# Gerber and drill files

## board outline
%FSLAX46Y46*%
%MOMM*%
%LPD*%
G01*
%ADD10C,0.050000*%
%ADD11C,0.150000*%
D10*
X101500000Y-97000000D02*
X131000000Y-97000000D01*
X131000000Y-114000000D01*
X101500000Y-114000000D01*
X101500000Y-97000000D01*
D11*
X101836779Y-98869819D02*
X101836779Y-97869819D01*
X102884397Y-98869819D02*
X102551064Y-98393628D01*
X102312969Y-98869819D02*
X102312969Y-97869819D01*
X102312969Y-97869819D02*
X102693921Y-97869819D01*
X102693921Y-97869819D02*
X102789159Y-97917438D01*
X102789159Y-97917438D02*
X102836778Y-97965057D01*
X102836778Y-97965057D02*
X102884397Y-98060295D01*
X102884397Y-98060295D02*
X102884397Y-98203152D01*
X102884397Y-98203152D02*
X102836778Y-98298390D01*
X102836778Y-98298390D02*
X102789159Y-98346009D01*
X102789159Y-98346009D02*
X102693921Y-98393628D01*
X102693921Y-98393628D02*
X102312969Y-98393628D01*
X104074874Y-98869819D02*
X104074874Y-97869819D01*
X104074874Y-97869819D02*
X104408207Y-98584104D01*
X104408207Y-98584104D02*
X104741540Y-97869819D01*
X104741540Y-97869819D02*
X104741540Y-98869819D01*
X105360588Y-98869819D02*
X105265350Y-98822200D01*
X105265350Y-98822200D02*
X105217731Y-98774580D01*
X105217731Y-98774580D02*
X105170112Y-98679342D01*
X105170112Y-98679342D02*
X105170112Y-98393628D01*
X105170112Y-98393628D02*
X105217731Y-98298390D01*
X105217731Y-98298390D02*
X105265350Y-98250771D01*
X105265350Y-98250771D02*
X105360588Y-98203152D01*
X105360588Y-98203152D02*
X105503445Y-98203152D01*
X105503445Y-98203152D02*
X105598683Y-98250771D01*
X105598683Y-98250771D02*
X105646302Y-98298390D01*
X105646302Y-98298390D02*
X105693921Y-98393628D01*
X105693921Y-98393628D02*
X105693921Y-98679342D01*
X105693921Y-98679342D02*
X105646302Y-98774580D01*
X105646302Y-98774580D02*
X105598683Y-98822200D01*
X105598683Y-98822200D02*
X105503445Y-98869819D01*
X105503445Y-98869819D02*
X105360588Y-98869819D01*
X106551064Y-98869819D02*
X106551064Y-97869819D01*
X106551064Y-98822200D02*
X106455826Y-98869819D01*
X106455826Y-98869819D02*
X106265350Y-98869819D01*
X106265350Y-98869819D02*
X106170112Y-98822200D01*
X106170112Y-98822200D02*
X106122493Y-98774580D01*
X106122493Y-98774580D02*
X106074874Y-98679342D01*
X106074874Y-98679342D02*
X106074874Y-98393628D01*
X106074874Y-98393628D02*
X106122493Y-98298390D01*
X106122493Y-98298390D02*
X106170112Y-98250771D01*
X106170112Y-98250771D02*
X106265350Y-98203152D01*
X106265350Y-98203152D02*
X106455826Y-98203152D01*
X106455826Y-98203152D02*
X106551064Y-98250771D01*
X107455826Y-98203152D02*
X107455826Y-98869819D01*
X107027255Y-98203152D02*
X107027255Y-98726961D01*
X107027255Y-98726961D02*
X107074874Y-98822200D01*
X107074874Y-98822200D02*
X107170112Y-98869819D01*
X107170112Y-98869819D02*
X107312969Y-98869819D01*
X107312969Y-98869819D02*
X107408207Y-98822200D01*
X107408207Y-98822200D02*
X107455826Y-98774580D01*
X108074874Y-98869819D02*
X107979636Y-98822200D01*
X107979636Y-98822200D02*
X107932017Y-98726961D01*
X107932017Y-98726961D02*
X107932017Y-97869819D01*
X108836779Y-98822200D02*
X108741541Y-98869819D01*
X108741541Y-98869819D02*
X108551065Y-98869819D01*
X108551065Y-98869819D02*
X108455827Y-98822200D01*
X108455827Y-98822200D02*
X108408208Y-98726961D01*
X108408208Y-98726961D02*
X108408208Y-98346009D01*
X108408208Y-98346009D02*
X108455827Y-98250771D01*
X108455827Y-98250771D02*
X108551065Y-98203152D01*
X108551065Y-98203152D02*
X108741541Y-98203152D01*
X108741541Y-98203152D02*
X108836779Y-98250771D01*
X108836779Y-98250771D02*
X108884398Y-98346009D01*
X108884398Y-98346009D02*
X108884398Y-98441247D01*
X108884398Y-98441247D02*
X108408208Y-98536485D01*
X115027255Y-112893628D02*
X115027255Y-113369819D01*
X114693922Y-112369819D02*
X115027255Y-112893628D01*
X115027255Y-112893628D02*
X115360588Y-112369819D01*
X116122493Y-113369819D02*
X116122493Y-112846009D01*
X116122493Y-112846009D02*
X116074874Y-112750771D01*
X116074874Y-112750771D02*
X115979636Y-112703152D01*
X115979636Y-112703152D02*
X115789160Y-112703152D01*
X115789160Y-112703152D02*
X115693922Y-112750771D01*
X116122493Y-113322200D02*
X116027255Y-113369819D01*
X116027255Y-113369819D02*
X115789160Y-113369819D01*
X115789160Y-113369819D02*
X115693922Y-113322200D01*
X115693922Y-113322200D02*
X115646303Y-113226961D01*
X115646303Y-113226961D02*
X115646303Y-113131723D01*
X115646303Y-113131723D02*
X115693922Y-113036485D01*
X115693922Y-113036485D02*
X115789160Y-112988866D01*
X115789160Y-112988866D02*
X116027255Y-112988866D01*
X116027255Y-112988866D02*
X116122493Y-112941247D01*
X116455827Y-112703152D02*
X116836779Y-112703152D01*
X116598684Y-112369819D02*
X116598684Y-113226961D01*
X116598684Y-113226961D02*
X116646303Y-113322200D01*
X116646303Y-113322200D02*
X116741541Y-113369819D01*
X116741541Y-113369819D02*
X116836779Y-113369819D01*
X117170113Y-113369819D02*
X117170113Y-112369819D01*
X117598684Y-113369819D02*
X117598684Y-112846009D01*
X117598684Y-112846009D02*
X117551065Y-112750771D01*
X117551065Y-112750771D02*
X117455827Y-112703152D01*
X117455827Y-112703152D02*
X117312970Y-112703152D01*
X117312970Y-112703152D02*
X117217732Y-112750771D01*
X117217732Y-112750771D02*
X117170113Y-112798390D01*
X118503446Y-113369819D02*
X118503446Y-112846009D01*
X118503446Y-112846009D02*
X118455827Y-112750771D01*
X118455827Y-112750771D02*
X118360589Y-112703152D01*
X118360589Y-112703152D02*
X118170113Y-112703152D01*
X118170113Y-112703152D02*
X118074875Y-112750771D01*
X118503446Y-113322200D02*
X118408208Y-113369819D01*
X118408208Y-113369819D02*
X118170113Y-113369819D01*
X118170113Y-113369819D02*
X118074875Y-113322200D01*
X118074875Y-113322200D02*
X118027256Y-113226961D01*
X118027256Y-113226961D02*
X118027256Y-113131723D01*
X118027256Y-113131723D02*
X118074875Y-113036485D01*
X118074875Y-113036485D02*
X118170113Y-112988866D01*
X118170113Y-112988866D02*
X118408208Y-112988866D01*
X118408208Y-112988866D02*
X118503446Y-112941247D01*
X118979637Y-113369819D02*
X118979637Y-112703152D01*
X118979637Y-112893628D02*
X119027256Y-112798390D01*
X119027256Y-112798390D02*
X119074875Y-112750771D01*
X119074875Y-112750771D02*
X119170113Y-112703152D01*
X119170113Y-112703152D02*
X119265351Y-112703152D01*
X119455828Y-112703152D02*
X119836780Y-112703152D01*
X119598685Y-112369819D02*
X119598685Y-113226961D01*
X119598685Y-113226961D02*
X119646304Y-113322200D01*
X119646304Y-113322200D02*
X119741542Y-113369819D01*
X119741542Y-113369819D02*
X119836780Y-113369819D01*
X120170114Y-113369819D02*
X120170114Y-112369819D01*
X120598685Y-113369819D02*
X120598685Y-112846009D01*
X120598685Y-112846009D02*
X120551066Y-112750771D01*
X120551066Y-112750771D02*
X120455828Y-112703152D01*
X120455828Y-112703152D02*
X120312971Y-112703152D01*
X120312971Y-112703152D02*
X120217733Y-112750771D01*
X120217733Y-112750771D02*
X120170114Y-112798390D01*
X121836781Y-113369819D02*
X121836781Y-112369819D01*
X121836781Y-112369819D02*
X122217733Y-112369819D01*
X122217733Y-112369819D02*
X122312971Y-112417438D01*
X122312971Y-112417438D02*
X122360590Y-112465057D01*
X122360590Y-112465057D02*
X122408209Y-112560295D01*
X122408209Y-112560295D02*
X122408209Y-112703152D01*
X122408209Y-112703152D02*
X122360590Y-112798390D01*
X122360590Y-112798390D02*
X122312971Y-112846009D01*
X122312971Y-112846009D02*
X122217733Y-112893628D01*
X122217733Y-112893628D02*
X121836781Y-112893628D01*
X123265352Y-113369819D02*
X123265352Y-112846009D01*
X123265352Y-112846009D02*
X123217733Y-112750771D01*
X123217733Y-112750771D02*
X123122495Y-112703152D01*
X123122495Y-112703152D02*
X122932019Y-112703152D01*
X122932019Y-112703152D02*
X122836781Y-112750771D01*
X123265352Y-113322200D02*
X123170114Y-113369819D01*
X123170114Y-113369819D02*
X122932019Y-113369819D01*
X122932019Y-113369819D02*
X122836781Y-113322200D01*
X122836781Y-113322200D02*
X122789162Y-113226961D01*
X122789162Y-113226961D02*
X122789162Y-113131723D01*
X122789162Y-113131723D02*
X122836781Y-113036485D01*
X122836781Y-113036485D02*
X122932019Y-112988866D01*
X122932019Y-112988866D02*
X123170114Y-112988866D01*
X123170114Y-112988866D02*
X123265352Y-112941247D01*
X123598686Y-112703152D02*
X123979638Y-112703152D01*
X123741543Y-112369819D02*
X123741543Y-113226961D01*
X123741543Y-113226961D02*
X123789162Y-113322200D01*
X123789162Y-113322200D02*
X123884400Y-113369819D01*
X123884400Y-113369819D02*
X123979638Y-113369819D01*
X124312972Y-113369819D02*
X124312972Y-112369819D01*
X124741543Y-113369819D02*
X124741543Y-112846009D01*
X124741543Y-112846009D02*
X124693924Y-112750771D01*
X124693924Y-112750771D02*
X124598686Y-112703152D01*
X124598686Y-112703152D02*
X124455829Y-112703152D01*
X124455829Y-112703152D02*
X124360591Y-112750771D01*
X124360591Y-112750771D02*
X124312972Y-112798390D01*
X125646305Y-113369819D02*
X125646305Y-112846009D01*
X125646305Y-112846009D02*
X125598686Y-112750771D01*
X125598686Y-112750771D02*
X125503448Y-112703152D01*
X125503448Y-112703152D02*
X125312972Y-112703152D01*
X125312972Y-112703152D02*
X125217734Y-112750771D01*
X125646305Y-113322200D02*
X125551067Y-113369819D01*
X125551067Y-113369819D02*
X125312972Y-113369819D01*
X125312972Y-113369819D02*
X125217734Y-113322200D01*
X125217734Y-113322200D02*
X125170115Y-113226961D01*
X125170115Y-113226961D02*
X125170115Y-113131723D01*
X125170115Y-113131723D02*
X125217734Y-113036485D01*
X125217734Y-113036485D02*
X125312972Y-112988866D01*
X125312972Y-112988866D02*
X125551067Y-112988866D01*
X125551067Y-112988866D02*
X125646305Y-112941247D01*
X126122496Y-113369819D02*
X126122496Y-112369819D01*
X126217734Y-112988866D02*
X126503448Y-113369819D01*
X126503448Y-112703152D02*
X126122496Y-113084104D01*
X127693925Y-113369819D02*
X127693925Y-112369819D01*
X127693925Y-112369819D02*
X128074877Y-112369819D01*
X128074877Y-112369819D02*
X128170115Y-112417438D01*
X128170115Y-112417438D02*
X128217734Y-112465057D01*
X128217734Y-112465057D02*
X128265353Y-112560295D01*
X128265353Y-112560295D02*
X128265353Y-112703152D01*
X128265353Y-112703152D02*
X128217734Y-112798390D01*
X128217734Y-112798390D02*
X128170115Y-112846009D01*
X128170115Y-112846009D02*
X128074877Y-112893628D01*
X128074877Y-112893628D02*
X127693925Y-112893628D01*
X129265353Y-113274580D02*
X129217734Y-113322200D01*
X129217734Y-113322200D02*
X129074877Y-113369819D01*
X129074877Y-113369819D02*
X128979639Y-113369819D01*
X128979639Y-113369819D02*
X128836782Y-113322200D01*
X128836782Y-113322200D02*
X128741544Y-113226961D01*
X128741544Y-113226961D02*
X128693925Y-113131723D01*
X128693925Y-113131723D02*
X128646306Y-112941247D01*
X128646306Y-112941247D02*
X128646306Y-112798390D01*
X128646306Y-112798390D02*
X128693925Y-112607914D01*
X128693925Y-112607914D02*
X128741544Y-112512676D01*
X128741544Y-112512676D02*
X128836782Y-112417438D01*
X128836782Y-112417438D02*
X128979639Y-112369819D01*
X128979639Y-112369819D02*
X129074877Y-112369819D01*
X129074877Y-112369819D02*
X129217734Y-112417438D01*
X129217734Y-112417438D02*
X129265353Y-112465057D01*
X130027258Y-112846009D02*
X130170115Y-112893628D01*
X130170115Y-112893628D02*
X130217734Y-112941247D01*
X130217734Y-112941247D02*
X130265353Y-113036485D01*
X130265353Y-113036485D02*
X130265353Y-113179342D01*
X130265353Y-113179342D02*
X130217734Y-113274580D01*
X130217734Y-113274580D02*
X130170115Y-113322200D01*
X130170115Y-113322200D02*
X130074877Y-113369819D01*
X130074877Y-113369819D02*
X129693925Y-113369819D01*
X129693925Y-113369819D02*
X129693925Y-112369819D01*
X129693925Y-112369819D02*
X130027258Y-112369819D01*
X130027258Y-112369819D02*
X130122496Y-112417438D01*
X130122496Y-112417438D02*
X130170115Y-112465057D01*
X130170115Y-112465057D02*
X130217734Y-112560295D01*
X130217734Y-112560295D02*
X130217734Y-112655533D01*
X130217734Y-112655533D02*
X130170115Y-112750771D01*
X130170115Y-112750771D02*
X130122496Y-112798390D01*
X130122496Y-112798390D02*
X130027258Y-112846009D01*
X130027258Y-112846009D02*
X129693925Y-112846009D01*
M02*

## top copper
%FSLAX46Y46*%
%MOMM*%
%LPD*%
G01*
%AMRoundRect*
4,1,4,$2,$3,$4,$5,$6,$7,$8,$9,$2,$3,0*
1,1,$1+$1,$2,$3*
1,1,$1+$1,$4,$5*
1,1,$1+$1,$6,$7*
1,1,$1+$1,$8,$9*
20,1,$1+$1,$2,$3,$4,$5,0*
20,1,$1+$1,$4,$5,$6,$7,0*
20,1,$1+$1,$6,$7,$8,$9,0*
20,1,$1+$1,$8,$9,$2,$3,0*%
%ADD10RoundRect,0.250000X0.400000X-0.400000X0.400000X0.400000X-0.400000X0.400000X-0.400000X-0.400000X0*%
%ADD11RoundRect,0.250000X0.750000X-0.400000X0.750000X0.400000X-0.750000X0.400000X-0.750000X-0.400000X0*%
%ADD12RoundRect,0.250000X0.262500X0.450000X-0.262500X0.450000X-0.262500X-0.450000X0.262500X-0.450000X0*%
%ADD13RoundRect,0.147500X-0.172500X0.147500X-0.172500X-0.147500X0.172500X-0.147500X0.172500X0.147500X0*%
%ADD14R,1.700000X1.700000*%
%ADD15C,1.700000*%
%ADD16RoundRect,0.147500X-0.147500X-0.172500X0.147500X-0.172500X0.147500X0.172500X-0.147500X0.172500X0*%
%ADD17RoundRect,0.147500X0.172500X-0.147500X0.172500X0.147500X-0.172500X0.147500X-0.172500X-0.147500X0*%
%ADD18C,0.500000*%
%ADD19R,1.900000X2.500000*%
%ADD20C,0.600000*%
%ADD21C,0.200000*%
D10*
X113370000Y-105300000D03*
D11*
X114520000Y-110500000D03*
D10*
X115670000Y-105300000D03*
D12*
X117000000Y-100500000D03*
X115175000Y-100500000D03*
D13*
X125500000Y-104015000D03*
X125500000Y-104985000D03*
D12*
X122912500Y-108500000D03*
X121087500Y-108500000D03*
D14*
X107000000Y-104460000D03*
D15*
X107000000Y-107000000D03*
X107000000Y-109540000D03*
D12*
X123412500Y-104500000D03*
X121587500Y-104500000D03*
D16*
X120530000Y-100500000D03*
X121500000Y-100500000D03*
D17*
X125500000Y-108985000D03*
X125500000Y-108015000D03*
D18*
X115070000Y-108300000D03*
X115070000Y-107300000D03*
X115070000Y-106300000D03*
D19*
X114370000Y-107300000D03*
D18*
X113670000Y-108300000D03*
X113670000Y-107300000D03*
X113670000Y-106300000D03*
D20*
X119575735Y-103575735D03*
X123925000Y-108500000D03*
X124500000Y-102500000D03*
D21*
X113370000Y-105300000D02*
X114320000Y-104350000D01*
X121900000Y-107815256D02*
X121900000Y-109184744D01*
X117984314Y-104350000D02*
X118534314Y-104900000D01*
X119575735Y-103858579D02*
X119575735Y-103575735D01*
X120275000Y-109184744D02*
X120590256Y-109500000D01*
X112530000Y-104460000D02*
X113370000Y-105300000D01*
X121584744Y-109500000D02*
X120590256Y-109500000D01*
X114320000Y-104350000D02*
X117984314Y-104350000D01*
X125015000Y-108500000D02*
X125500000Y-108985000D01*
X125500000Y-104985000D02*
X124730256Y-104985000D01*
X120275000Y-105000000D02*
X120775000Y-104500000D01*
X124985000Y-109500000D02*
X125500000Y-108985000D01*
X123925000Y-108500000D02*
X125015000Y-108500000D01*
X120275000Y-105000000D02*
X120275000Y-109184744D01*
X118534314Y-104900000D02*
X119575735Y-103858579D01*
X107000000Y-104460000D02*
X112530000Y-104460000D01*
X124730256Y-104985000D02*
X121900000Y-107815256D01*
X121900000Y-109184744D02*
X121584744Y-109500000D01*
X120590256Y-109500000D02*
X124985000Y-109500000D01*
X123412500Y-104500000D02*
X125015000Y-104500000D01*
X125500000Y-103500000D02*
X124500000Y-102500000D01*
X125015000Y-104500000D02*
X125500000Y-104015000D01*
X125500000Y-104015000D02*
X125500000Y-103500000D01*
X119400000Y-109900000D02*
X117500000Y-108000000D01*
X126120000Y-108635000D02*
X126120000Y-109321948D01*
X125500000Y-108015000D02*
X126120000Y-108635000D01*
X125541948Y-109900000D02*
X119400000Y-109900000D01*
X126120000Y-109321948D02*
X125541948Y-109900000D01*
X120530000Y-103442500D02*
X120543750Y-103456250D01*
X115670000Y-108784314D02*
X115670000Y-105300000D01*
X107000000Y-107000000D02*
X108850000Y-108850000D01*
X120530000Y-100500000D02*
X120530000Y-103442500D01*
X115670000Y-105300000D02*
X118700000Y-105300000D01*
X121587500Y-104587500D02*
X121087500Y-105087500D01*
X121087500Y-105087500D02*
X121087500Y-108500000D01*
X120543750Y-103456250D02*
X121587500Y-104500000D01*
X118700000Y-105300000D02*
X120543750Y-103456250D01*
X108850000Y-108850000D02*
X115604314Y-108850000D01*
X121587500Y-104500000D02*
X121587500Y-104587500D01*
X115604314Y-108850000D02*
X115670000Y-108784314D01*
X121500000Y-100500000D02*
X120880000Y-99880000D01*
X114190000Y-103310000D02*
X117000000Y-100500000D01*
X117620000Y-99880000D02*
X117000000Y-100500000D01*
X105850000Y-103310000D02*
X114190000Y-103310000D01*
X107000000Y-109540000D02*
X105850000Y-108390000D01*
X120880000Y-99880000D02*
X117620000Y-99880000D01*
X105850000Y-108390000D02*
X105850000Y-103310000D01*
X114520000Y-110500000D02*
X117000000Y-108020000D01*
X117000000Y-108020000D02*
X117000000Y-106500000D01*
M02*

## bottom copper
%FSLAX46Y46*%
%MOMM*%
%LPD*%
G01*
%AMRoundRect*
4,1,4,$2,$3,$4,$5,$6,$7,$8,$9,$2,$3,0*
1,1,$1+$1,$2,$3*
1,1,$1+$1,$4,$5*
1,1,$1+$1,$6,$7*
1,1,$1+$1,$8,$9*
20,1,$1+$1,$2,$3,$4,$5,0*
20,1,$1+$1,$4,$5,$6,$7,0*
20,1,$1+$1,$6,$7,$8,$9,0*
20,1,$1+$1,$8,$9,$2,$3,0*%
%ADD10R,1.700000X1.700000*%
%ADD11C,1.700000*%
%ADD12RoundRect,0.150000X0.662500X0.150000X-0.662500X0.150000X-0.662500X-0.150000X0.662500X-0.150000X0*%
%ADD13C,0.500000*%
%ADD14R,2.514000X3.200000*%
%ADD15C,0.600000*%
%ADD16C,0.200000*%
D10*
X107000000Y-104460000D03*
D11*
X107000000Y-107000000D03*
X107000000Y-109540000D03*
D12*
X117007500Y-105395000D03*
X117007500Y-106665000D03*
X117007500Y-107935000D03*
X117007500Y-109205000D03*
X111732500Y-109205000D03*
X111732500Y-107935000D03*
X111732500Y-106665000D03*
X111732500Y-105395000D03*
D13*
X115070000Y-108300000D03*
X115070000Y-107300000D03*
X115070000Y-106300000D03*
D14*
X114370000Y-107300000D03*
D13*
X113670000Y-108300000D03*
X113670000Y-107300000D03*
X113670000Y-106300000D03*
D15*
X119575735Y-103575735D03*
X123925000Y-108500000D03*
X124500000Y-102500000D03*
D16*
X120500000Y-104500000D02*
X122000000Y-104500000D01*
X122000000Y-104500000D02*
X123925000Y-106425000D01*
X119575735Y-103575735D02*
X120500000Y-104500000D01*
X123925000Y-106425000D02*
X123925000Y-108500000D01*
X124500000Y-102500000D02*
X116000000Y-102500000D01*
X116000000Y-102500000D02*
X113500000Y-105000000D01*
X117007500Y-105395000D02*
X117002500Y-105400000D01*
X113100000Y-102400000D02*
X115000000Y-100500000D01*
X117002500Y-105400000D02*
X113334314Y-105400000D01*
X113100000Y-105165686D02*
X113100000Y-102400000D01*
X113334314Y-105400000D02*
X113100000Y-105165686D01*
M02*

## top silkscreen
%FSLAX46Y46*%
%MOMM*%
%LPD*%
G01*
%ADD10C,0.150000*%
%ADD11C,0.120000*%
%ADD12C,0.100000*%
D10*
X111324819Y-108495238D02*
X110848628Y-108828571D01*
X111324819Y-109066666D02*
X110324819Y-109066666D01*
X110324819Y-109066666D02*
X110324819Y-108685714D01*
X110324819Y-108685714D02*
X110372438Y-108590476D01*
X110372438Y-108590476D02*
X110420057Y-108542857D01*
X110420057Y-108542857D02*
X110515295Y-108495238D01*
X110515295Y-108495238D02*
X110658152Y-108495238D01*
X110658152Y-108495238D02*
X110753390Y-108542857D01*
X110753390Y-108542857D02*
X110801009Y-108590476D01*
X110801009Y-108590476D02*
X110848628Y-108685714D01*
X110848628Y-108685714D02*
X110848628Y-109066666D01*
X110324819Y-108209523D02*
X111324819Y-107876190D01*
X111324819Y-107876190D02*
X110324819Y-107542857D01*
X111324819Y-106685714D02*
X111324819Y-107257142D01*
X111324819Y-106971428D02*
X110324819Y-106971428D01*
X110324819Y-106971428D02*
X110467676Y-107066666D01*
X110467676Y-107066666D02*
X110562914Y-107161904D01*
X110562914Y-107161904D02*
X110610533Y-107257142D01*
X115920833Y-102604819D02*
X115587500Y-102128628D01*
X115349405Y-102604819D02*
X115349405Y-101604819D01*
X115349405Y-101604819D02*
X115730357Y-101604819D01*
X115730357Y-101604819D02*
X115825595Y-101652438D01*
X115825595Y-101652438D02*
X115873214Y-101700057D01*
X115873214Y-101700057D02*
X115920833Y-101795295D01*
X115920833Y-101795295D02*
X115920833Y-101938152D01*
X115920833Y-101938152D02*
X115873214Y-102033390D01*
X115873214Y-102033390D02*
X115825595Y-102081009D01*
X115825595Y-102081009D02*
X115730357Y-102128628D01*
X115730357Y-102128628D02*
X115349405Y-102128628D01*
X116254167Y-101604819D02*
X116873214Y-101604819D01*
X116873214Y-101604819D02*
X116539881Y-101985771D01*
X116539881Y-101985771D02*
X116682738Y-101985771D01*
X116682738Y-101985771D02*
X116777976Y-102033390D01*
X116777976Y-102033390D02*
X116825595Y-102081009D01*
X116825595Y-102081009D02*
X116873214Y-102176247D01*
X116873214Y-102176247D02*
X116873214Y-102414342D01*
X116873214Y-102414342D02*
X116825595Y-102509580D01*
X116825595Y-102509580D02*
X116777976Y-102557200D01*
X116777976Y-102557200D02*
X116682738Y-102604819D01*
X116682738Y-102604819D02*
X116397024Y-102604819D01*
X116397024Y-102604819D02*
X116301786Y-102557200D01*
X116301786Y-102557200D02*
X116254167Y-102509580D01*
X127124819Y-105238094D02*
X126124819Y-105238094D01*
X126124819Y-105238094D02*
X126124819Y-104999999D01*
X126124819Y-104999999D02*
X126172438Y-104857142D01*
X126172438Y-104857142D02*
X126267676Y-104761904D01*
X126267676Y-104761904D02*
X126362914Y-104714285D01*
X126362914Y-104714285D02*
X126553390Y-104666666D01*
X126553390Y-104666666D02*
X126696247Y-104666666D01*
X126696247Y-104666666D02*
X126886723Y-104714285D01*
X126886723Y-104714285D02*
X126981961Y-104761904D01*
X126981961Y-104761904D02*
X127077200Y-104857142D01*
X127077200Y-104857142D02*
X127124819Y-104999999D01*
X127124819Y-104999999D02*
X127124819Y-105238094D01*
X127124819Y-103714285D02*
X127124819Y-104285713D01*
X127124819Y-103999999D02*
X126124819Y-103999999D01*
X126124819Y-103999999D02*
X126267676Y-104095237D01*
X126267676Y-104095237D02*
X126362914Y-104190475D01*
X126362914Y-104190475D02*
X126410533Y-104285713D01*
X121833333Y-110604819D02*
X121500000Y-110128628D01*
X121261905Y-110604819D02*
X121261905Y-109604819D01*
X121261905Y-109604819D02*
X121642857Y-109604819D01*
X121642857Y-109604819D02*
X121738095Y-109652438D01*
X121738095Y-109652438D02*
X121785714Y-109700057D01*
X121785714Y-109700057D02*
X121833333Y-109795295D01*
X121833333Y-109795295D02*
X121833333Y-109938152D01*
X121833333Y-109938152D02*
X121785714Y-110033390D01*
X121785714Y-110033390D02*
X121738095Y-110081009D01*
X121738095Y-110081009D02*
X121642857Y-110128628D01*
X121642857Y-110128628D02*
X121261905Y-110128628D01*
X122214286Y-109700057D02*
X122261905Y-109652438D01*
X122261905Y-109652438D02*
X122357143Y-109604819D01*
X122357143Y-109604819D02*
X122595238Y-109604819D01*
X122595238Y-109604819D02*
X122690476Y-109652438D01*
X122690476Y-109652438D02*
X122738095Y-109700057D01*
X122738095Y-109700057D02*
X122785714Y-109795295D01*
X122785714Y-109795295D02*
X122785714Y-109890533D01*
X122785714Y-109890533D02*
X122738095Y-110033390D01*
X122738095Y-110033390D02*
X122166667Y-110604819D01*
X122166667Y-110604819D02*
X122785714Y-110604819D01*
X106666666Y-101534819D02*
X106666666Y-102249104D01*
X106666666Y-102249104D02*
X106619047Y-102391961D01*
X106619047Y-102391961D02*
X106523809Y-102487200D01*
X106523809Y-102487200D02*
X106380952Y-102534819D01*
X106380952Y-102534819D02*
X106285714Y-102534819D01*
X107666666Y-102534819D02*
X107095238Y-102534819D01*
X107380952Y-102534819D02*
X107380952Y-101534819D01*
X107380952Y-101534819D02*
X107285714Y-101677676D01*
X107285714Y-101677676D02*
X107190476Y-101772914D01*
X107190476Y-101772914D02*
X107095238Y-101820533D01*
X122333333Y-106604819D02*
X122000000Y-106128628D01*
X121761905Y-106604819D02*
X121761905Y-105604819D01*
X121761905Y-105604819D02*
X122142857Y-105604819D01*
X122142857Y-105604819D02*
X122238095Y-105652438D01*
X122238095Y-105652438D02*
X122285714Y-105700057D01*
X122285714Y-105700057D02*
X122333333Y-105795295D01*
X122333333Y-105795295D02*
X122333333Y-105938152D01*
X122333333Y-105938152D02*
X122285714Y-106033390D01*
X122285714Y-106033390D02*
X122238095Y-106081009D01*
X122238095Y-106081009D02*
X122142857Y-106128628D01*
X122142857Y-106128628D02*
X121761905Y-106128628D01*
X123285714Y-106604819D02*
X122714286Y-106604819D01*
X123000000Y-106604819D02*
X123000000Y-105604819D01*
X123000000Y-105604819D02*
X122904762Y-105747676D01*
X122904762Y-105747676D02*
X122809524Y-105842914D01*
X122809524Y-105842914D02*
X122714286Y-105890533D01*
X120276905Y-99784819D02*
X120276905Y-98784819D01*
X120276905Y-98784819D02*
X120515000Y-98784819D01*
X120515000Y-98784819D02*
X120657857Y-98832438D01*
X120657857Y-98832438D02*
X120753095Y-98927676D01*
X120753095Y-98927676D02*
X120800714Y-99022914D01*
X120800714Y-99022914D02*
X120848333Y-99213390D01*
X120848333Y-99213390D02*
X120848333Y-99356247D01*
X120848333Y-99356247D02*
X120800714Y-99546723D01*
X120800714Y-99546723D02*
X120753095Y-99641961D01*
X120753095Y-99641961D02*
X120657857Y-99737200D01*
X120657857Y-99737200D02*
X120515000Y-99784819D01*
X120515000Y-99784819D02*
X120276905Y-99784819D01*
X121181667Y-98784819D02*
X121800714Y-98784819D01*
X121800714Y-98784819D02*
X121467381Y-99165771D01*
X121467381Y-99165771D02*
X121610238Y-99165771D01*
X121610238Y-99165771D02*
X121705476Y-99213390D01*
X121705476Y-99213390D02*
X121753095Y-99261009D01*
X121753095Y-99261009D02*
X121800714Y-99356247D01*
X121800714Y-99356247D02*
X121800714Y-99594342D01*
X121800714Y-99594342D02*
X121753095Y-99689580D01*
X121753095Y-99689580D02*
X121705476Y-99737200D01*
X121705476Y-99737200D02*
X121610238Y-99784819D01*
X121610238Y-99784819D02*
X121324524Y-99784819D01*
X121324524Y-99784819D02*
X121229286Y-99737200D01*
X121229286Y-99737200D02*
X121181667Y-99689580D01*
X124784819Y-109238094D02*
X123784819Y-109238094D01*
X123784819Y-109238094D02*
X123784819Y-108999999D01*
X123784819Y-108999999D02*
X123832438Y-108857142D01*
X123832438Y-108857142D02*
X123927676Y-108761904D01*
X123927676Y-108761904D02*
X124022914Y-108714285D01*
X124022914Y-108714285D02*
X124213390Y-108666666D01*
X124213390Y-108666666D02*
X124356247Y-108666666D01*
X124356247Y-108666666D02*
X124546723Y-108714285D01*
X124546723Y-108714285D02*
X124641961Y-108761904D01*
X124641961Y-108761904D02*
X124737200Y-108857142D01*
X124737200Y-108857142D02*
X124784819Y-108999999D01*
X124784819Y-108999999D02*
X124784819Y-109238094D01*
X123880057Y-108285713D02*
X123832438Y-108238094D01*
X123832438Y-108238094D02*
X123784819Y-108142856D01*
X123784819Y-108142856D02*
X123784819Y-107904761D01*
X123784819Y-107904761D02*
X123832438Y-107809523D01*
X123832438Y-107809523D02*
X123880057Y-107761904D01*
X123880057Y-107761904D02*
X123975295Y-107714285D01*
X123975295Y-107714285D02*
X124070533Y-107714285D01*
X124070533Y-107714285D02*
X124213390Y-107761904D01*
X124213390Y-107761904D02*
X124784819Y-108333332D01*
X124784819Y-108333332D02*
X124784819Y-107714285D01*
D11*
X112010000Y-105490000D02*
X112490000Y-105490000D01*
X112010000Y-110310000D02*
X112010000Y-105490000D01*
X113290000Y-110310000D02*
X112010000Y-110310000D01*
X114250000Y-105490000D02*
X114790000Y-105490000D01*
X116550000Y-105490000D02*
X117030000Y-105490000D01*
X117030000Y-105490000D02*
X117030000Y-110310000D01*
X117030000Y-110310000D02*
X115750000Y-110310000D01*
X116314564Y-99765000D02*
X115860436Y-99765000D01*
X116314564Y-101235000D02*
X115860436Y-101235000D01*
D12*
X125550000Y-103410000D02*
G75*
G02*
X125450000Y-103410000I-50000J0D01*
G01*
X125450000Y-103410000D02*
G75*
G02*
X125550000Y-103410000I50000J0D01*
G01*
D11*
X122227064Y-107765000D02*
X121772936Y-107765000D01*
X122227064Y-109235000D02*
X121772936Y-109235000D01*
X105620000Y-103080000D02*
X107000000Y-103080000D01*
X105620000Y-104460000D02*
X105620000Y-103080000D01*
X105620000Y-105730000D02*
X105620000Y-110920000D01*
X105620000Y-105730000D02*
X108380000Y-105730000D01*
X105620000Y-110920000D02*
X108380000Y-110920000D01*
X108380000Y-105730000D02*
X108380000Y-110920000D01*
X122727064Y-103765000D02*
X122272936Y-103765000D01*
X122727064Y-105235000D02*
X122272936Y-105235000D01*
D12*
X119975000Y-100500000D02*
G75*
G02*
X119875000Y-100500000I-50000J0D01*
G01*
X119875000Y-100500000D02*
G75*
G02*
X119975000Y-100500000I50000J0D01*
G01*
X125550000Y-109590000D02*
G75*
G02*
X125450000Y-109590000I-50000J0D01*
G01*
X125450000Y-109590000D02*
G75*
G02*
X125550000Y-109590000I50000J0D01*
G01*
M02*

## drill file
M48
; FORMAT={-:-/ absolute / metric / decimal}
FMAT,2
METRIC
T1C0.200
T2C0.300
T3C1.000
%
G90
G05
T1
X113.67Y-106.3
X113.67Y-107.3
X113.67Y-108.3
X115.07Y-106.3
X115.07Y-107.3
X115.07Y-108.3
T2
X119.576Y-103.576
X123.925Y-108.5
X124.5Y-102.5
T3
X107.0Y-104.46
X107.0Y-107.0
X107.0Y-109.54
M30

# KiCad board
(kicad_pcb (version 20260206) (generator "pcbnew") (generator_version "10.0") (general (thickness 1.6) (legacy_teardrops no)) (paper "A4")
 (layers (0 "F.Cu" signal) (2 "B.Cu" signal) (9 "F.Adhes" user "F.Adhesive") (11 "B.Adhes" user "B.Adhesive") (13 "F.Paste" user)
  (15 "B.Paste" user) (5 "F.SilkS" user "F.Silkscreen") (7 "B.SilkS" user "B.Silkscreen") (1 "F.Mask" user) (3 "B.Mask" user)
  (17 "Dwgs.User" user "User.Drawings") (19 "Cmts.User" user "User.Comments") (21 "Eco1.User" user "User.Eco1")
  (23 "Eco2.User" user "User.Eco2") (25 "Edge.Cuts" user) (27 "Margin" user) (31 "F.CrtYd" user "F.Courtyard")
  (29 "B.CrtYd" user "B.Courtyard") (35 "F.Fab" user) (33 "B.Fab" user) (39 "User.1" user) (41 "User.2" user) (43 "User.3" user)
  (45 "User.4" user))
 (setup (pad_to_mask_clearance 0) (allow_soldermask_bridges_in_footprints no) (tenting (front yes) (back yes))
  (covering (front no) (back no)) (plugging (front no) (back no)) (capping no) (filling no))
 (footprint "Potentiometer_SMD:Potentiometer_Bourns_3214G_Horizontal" (layer "F.Cu") (at 114.52 107.9 90)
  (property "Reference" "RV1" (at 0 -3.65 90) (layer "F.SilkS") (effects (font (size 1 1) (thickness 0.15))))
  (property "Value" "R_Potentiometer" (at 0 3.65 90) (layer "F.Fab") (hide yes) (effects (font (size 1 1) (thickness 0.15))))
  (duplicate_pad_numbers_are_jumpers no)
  (fp_line (start 2.41 -2.51) (end 2.41 -2.03) (stroke (width 0.12) (type solid)) (layer "F.SilkS"))
  (fp_line (start -2.41 -2.51) (end 2.41 -2.51) (stroke (width 0.12) (type solid)) (layer "F.SilkS"))
  (fp_line (start -2.41 -1.23) (end -2.41 -2.51) (stroke (width 0.12) (type solid)) (layer "F.SilkS"))
  (fp_line (start 2.41 -0.27) (end 2.41 0.27) (stroke (width 0.12) (type solid)) (layer "F.SilkS"))
  (fp_line (start 2.41 2.03) (end 2.41 2.51) (stroke (width 0.12) (type solid)) (layer "F.SilkS"))
  (fp_line (start 2.41 2.51) (end -2.41 2.51) (stroke (width 0.12) (type solid)) (layer "F.SilkS"))
  (fp_line (start -2.41 2.51) (end -2.41 1.23) (stroke (width 0.12) (type solid)) (layer "F.SilkS"))
  (pad "1" smd roundrect (at 2.6 -1.15 90) (size 1.3 1.3) (layers "F.Cu" "F.Mask" "F.Paste") (roundrect_rratio 0.192308) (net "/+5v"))
  (pad "2" smd roundrect (at -2.6 0 90) (size 1.3 2) (layers "F.Cu" "F.Mask" "F.Paste") (roundrect_rratio 0.192308) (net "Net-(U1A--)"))
  (pad "3" smd roundrect (at 2.6 1.15 90) (size 1.3 1.3) (layers "F.Cu" "F.Mask" "F.Paste") (roundrect_rratio 0.192308) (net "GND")))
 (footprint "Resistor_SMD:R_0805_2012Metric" (layer "F.Cu") (at 116.0875 100.5 180)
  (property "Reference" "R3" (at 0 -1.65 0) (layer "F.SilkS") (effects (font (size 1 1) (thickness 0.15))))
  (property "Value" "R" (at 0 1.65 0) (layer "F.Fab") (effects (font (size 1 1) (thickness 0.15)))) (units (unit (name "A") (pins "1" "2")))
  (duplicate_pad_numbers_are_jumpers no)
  (fp_line (start -0.227064 0.735) (end 0.227064 0.735) (stroke (width 0.12) (type solid)) (layer "F.SilkS"))
  (fp_line (start -0.227064 -0.735) (end 0.227064 -0.735) (stroke (width 0.12) (type solid)) (layer "F.SilkS"))
  (pad "1" smd roundrect (at -0.9125 0 180) (size 1.025 1.4) (layers "F.Cu" "F.Mask" "F.Paste") (roundrect_rratio 0.243902)
   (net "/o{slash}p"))
  (pad "2" smd roundrect (at 0.9125 0 180) (size 1.025 1.4) (layers "F.Cu" "F.Mask" "F.Paste") (roundrect_rratio 0.243902)
   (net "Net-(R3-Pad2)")))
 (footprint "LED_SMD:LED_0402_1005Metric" (layer "F.Cu") (at 125.5 104.5 -90)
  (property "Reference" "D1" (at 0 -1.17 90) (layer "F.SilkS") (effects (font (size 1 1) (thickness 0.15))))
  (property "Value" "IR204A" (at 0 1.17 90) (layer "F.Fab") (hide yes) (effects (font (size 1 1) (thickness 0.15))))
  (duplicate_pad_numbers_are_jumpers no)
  (fp_circle (center -1.09 0) (end -1.04 0) (stroke (width 0.1) (type solid)) (fill no) (layer "F.SilkS"))
  (pad "1" smd roundrect (at -0.485 0 270) (size 0.59 0.64) (layers "F.Cu" "F.Mask" "F.Paste") (roundrect_rratio 0.25) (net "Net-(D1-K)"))
  (pad "2" smd roundrect (at 0.485 0 270) (size 0.59 0.64) (layers "F.Cu" "F.Mask" "F.Paste") (roundrect_rratio 0.25) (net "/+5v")))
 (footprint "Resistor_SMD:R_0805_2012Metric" (layer "F.Cu") (at 122 108.5 180)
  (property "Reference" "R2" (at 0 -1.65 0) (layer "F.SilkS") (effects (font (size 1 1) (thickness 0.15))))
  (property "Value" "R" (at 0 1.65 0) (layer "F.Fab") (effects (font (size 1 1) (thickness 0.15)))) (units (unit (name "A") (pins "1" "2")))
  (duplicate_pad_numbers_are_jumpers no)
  (fp_line (start -0.227064 0.735) (end 0.227064 0.735) (stroke (width 0.12) (type solid)) (layer "F.SilkS"))
  (fp_line (start -0.227064 -0.735) (end 0.227064 -0.735) (stroke (width 0.12) (type solid)) (layer "F.SilkS"))
  (pad "1" smd roundrect (at -0.9125 0 180) (size 1.025 1.4) (layers "F.Cu" "F.Mask" "F.Paste") (roundrect_rratio 0.243902)
   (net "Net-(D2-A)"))
  (pad "2" smd roundrect (at 0.9125 0 180) (size 1.025 1.4) (layers "F.Cu" "F.Mask" "F.Paste") (roundrect_rratio 0.243902) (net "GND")))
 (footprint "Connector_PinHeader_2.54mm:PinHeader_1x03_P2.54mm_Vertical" (layer "F.Cu") (at 107 104.46)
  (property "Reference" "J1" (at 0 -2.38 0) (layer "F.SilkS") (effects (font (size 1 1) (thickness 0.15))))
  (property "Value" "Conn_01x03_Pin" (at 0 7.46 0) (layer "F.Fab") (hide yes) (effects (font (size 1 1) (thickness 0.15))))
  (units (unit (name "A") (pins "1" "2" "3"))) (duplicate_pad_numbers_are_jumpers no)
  (fp_line (start -1.38 -1.38) (end 0 -1.38) (stroke (width 0.12) (type solid)) (layer "F.SilkS"))
  (fp_line (start -1.38 0) (end -1.38 -1.38) (stroke (width 0.12) (type solid)) (layer "F.SilkS"))
  (fp_line (start -1.38 1.27) (end -1.38 6.46) (stroke (width 0.12) (type solid)) (layer "F.SilkS"))
  (fp_line (start -1.38 1.27) (end 1.38 1.27) (stroke (width 0.12) (type solid)) (layer "F.SilkS"))
  (fp_line (start -1.38 6.46) (end 1.38 6.46) (stroke (width 0.12) (type solid)) (layer "F.SilkS"))
  (fp_line (start 1.38 1.27) (end 1.38 6.46) (stroke (width 0.12) (type solid)) (layer "F.SilkS"))
  (pad "1" thru_hole rect (at 0 0) (size 1.7 1.7) (drill 1) (layers "*.Cu" "*.Mask") (remove_unused_layers no) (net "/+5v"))
  (pad "2" thru_hole circle (at 0 2.54) (size 1.7 1.7) (drill 1) (layers "*.Cu" "*.Mask") (remove_unused_layers no) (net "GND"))
  (pad "3" thru_hole circle (at 0 5.08) (size 1.7 1.7) (drill 1) (layers "*.Cu" "*.Mask") (remove_unused_layers no) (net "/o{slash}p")))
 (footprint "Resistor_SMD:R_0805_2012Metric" (layer "F.Cu") (at 122.5 104.5 180)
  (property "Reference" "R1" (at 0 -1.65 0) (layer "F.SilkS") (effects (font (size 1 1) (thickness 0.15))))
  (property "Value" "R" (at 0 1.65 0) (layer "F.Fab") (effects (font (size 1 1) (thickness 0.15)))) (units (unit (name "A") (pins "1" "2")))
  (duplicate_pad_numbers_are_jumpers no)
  (fp_line (start -0.227064 0.735) (end 0.227064 0.735) (stroke (width 0.12) (type solid)) (layer "F.SilkS"))
  (fp_line (start -0.227064 -0.735) (end 0.227064 -0.735) (stroke (width 0.12) (type solid)) (layer "F.SilkS"))
  (pad "1" smd roundrect (at -0.9125 0 180) (size 1.025 1.4) (layers "F.Cu" "F.Mask" "F.Paste") (roundrect_rratio 0.243902)
   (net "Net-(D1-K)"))
  (pad "2" smd roundrect (at 0.9125 0 180) (size 1.025 1.4) (layers "F.Cu" "F.Mask" "F.Paste") (roundrect_rratio 0.243902) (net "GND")))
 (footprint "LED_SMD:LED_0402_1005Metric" (layer "F.Cu") (at 121.015 100.5)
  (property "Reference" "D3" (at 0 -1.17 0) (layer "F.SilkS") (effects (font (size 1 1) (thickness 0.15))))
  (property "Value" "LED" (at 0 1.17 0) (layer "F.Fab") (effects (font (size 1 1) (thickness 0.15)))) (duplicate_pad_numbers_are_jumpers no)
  (fp_circle (center -1.09 0) (end -1.04 0) (stroke (width 0.1) (type solid)) (fill no) (layer "F.SilkS"))
  (pad "1" smd roundrect (at -0.485 0) (size 0.59 0.64) (layers "F.Cu" "F.Mask" "F.Paste") (roundrect_rratio 0.25) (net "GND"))
  (pad "2" smd roundrect (at 0.485 0) (size 0.59 0.64) (layers "F.Cu" "F.Mask" "F.Paste") (roundrect_rratio 0.25) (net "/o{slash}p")))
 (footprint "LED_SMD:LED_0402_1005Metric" (layer "F.Cu") (at 125.5 108.5 90)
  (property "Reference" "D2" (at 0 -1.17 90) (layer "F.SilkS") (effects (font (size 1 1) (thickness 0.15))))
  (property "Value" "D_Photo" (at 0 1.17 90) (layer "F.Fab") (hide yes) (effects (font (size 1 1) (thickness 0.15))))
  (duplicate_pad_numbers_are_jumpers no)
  (fp_circle (center -1.09 0) (end -1.04 0) (stroke (width 0.1) (type solid)) (fill no) (layer "F.SilkS"))
  (pad "1" smd roundrect (at -0.485 0 90) (size 0.59 0.64) (layers "F.Cu" "F.Mask" "F.Paste") (roundrect_rratio 0.25) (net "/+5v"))
  (pad "2" smd roundrect (at 0.485 0 90) (size 0.59 0.64) (layers "F.Cu" "F.Mask" "F.Paste") (roundrect_rratio 0.25) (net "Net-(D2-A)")))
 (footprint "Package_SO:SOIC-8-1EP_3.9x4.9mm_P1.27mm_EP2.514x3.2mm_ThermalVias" (layer "B.Cu") (at 114.37 107.3 180)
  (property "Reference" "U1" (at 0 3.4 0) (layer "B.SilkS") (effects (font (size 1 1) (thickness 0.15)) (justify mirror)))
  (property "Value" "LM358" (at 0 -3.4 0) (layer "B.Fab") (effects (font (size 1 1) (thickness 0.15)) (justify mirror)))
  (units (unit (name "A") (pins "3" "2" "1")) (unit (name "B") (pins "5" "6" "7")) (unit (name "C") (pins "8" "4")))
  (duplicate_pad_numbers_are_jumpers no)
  (pad "" smd roundrect (at -0.63 -0.8 180) (size 1.05 1.34) (layers "B.Paste") (roundrect_rratio 0.238095))
  (pad "" smd roundrect (at -0.63 0.8 180) (size 1.05 1.34) (layers "B.Paste") (roundrect_rratio 0.238095))
  (pad "" smd roundrect (at 0.63 -0.8 180) (size 1.05 1.34) (layers "B.Paste") (roundrect_rratio 0.238095))
  (pad "" smd roundrect (at 0.63 0.8 180) (size 1.05 1.34) (layers "B.Paste") (roundrect_rratio 0.238095))
  (pad "1" smd roundrect (at -2.6375 1.905 180) (size 1.625 0.6) (layers "B.Cu" "B.Mask" "B.Paste") (roundrect_rratio 0.25)
   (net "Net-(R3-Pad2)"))
  (pad "2" smd roundrect (at -2.6375 0.635 180) (size 1.625 0.6) (layers "B.Cu" "B.Mask" "B.Paste") (roundrect_rratio 0.25)
   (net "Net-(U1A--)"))
  (pad "3" smd roundrect (at -2.6375 -0.635 180) (size 1.625 0.6) (layers "B.Cu" "B.Mask" "B.Paste") (roundrect_rratio 0.25)
   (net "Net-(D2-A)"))
  (pad "4" smd roundrect (at -2.6375 -1.905 180) (size 1.625 0.6) (layers "B.Cu" "B.Mask" "B.Paste") (roundrect_rratio 0.25))
  (pad "5" smd roundrect (at 2.6375 -1.905 180) (size 1.625 0.6) (layers "B.Cu" "B.Mask" "B.Paste") (roundrect_rratio 0.25))
  (pad "6" smd roundrect (at 2.6375 -0.635 180) (size 1.625 0.6) (layers "B.Cu" "B.Mask" "B.Paste") (roundrect_rratio 0.25))
  (pad "7" smd roundrect (at 2.6375 0.635 180) (size 1.625 0.6) (layers "B.Cu" "B.Mask" "B.Paste") (roundrect_rratio 0.25))
  (pad "8" smd roundrect (at 2.6375 1.905 180) (size 1.625 0.6) (layers "B.Cu" "B.Mask" "B.Paste") (roundrect_rratio 0.25))
  (pad "9" thru_hole circle (at -0.7 -1 180) (size 0.5 0.5) (drill 0.2) (layers "*.Cu") (remove_unused_layers no))
  (pad "9" thru_hole circle (at -0.7 0 180) (size 0.5 0.5) (drill 0.2) (layers "*.Cu") (remove_unused_layers no))
  (pad "9" thru_hole circle (at -0.7 1 180) (size 0.5 0.5) (drill 0.2) (layers "*.Cu") (remove_unused_layers no))
  (pad "9" smd rect (at 0 0 180) (size 1.9 2.5) (layers "F.Cu") (zone_connect 2))
  (pad "9" smd rect (at 0 0 180) (size 2.514 3.2) (layers "B.Cu" "B.Mask") (zone_connect 2))
  (pad "9" thru_hole circle (at 0.7 -1 180) (size 0.5 0.5) (drill 0.2) (layers "*.Cu") (remove_unused_layers no))
  (pad "9" thru_hole circle (at 0.7 0 180) (size 0.5 0.5) (drill 0.2) (layers "*.Cu") (remove_unused_layers no))
  (pad "9" thru_hole circle (at 0.7 1 180) (size 0.5 0.5) (drill 0.2) (layers "*.Cu") (remove_unused_layers no)))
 (gr_rect (start 101.5 97) (end 131 114) (stroke (width 0.05) (type default)) (fill no) (layer "Edge.Cuts"))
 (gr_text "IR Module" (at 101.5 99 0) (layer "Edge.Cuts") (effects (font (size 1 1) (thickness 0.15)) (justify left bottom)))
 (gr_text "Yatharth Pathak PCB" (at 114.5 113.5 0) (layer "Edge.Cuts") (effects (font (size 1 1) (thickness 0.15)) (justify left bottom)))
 (segment (start 113.37 105.3) (end 114.32 104.35) (width 0.2) (layer "F.Cu") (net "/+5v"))
 (segment (start 121.9 107.815256) (end 121.9 109.184744) (width 0.2) (layer "F.Cu") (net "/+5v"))
 (segment (start 117.984314 104.35) (end 118.534314 104.9) (width 0.2) (layer "F.Cu") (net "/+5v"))
 (segment (start 119.575735 103.858579) (end 119.575735 103.575735) (width 0.2) (layer "F.Cu") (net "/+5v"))
 (segment (start 120.275 109.184744) (end 120.590256 109.5) (width 0.2) (layer "F.Cu") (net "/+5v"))
 (segment (start 112.53 104.46) (end 113.37 105.3) (width 0.2) (layer "F.Cu") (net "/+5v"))
 (segment (start 121.584744 109.5) (end 120.590256 109.5) (width 0.2) (layer "F.Cu") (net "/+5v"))
 (segment (start 114.32 104.35) (end 117.984314 104.35) (width 0.2) (layer "F.Cu") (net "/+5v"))
 (segment (start 125.015 108.5) (end 125.5 108.985) (width 0.2) (layer "F.Cu") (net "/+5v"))
 (segment (start 125.5 104.985) (end 124.730256 104.985) (width 0.2) (layer "F.Cu") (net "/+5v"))
 (segment (start 120.275 105) (end 120.775 104.5) (width 0.2) (layer "F.Cu") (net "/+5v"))
 (segment (start 124.985 109.5) (end 125.5 108.985) (width 0.2) (layer "F.Cu") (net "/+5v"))
 (segment (start 123.925 108.5) (end 125.015 108.5) (width 0.2) (layer "F.Cu") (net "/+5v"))
 (segment (start 120.275 105) (end 120.275 109.184744) (width 0.2) (layer "F.Cu") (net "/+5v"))
 (segment (start 118.534314 104.9) (end 119.575735 103.858579) (width 0.2) (layer "F.Cu") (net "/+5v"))
 (segment (start 107 104.46) (end 112.53 104.46) (width 0.2) (layer "F.Cu") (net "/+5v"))
 (segment (start 124.730256 104.985) (end 121.9 107.815256) (width 0.2) (layer "F.Cu") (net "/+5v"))
 (segment (start 121.9 109.184744) (end 121.584744 109.5) (width 0.2) (layer "F.Cu") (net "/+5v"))
 (segment (start 120.590256 109.5) (end 124.985 109.5) (width 0.2) (layer "F.Cu") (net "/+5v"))
 (via (at 119.575735 103.575735) (size 0.6) (drill 0.3) (layers "F.Cu" "B.Cu") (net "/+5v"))
 (via (at 123.925 108.5) (size 0.6) (drill 0.3) (layers "F.Cu" "B.Cu") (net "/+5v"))
 (segment (start 120.5 104.5) (end 122 104.5) (width 0.2) (layer "B.Cu") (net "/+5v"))
 (segment (start 122 104.5) (end 123.925 106.425) (width 0.2) (layer "B.Cu") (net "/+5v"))
 (segment (start 119.575735 103.575735) (end 120.5 104.5) (width 0.2) (layer "B.Cu") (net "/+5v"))
 (segment (start 123.925 106.425) (end 123.925 108.5) (width 0.2) (layer "B.Cu") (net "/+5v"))
 (segment (start 123.4125 104.5) (end 125.015 104.5) (width 0.2) (layer "F.Cu") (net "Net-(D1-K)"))
 (segment (start 125.5 103.5) (end 124.5 102.5) (width 0.2) (layer "F.Cu") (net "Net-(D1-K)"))
 (segment (start 125.015 104.5) (end 125.5 104.015) (width 0.2) (layer "F.Cu") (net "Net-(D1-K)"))
 (segment (start 125.5 104.015) (end 125.5 103.5) (width 0.2) (layer "F.Cu") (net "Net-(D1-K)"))
 (via (at 124.5 102.5) (size 0.6) (drill 0.3) (layers "F.Cu" "B.Cu") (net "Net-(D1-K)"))
 (segment (start 124.5 102.5) (end 116 102.5) (width 0.2) (layer "B.Cu") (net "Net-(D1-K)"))
 (segment (start 116 102.5) (end 113.5 105) (width 0.2) (layer "B.Cu") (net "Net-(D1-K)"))
 (segment (start 119.4 109.9) (end 117.5 108) (width 0.2) (layer "F.Cu") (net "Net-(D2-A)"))
 (segment (start 126.12 108.635) (end 126.12 109.321948) (width 0.2) (layer "F.Cu") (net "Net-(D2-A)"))
 (segment (start 125.5 108.015) (end 126.12 108.635) (width 0.2) (layer "F.Cu") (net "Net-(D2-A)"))
 (segment (start 125.541948 109.9) (end 119.4 109.9) (width 0.2) (layer "F.Cu") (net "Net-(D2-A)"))
 (segment (start 126.12 109.321948) (end 125.541948 109.9) (width 0.2) (layer "F.Cu") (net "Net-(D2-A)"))
 (segment (start 120.53 103.4425) (end 120.54375 103.45625) (width 0.2) (layer "F.Cu") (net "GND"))
 (segment (start 115.67 108.784314) (end 115.67 105.3) (width 0.2) (layer "F.Cu") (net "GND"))
 (segment (start 107 107) (end 108.85 108.85) (width 0.2) (layer "F.Cu") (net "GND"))
 (segment (start 120.53 100.5) (end 120.53 103.4425) (width 0.2) (layer "F.Cu") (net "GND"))
 (segment (start 115.67 105.3) (end 118.7 105.3) (width 0.2) (layer "F.Cu") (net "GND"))
 (segment (start 121.5875 104.5875) (end 121.0875 105.0875) (width 0.2) (layer "F.Cu") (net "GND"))
 (segment (start 121.0875 105.0875) (end 121.0875 108.5) (width 0.2) (layer "F.Cu") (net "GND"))
 (segment (start 120.54375 103.45625) (end 121.5875 104.5) (width 0.2) (layer "F.Cu") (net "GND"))
 (segment (start 118.7 105.3) (end 120.54375 103.45625) (width 0.2) (layer "F.Cu") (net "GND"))
 (segment (start 108.85 108.85) (end 115.604314 108.85) (width 0.2) (layer "F.Cu") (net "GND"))
 (segment (start 121.5875 104.5) (end 121.5875 104.5875) (width 0.2) (layer "F.Cu") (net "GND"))
 (segment (start 115.604314 108.85) (end 115.67 108.784314) (width 0.2) (layer "F.Cu") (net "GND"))
 (segment (start 121.5 100.5) (end 120.88 99.88) (width 0.2) (layer "F.Cu") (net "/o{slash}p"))
 (segment (start 114.19 103.31) (end 117 100.5) (width 0.2) (layer "F.Cu") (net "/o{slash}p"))
 (segment (start 117.62 99.88) (end 117 100.5) (width 0.2) (layer "F.Cu") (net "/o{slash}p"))
 (segment (start 105.85 103.31) (end 114.19 103.31) (width 0.2) (layer "F.Cu") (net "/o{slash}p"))
 (segment (start 107 109.54) (end 105.85 108.39) (width 0.2) (layer "F.Cu") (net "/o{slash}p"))
 (segment (start 120.88 99.88) (end 117.62 99.88) (width 0.2) (layer "F.Cu") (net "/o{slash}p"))
 (segment (start 105.85 108.39) (end 105.85 103.31) (width 0.2) (layer "F.Cu") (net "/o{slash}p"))
 (segment (start 117.0075 105.395) (end 117.0025 105.4) (width 0.2) (layer "B.Cu") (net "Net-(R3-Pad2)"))
 (segment (start 113.1 102.4) (end 115 100.5) (width 0.2) (layer "B.Cu") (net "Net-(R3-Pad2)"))
 (segment (start 117.0025 105.4) (end 113.334314 105.4) (width 0.2) (layer "B.Cu") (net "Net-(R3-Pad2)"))
 (segment (start 113.1 105.165686) (end 113.1 102.4) (width 0.2) (layer "B.Cu") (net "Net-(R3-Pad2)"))
 (segment (start 113.334314 105.4) (end 113.1 105.165686) (width 0.2) (layer "B.Cu") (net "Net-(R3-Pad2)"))
 (segment (start 114.52 110.5) (end 117 108.02) (width 0.2) (layer "F.Cu") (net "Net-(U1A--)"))
 (segment (start 117 108.02) (end 117 106.5) (width 0.2) (layer "F.Cu") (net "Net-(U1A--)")))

